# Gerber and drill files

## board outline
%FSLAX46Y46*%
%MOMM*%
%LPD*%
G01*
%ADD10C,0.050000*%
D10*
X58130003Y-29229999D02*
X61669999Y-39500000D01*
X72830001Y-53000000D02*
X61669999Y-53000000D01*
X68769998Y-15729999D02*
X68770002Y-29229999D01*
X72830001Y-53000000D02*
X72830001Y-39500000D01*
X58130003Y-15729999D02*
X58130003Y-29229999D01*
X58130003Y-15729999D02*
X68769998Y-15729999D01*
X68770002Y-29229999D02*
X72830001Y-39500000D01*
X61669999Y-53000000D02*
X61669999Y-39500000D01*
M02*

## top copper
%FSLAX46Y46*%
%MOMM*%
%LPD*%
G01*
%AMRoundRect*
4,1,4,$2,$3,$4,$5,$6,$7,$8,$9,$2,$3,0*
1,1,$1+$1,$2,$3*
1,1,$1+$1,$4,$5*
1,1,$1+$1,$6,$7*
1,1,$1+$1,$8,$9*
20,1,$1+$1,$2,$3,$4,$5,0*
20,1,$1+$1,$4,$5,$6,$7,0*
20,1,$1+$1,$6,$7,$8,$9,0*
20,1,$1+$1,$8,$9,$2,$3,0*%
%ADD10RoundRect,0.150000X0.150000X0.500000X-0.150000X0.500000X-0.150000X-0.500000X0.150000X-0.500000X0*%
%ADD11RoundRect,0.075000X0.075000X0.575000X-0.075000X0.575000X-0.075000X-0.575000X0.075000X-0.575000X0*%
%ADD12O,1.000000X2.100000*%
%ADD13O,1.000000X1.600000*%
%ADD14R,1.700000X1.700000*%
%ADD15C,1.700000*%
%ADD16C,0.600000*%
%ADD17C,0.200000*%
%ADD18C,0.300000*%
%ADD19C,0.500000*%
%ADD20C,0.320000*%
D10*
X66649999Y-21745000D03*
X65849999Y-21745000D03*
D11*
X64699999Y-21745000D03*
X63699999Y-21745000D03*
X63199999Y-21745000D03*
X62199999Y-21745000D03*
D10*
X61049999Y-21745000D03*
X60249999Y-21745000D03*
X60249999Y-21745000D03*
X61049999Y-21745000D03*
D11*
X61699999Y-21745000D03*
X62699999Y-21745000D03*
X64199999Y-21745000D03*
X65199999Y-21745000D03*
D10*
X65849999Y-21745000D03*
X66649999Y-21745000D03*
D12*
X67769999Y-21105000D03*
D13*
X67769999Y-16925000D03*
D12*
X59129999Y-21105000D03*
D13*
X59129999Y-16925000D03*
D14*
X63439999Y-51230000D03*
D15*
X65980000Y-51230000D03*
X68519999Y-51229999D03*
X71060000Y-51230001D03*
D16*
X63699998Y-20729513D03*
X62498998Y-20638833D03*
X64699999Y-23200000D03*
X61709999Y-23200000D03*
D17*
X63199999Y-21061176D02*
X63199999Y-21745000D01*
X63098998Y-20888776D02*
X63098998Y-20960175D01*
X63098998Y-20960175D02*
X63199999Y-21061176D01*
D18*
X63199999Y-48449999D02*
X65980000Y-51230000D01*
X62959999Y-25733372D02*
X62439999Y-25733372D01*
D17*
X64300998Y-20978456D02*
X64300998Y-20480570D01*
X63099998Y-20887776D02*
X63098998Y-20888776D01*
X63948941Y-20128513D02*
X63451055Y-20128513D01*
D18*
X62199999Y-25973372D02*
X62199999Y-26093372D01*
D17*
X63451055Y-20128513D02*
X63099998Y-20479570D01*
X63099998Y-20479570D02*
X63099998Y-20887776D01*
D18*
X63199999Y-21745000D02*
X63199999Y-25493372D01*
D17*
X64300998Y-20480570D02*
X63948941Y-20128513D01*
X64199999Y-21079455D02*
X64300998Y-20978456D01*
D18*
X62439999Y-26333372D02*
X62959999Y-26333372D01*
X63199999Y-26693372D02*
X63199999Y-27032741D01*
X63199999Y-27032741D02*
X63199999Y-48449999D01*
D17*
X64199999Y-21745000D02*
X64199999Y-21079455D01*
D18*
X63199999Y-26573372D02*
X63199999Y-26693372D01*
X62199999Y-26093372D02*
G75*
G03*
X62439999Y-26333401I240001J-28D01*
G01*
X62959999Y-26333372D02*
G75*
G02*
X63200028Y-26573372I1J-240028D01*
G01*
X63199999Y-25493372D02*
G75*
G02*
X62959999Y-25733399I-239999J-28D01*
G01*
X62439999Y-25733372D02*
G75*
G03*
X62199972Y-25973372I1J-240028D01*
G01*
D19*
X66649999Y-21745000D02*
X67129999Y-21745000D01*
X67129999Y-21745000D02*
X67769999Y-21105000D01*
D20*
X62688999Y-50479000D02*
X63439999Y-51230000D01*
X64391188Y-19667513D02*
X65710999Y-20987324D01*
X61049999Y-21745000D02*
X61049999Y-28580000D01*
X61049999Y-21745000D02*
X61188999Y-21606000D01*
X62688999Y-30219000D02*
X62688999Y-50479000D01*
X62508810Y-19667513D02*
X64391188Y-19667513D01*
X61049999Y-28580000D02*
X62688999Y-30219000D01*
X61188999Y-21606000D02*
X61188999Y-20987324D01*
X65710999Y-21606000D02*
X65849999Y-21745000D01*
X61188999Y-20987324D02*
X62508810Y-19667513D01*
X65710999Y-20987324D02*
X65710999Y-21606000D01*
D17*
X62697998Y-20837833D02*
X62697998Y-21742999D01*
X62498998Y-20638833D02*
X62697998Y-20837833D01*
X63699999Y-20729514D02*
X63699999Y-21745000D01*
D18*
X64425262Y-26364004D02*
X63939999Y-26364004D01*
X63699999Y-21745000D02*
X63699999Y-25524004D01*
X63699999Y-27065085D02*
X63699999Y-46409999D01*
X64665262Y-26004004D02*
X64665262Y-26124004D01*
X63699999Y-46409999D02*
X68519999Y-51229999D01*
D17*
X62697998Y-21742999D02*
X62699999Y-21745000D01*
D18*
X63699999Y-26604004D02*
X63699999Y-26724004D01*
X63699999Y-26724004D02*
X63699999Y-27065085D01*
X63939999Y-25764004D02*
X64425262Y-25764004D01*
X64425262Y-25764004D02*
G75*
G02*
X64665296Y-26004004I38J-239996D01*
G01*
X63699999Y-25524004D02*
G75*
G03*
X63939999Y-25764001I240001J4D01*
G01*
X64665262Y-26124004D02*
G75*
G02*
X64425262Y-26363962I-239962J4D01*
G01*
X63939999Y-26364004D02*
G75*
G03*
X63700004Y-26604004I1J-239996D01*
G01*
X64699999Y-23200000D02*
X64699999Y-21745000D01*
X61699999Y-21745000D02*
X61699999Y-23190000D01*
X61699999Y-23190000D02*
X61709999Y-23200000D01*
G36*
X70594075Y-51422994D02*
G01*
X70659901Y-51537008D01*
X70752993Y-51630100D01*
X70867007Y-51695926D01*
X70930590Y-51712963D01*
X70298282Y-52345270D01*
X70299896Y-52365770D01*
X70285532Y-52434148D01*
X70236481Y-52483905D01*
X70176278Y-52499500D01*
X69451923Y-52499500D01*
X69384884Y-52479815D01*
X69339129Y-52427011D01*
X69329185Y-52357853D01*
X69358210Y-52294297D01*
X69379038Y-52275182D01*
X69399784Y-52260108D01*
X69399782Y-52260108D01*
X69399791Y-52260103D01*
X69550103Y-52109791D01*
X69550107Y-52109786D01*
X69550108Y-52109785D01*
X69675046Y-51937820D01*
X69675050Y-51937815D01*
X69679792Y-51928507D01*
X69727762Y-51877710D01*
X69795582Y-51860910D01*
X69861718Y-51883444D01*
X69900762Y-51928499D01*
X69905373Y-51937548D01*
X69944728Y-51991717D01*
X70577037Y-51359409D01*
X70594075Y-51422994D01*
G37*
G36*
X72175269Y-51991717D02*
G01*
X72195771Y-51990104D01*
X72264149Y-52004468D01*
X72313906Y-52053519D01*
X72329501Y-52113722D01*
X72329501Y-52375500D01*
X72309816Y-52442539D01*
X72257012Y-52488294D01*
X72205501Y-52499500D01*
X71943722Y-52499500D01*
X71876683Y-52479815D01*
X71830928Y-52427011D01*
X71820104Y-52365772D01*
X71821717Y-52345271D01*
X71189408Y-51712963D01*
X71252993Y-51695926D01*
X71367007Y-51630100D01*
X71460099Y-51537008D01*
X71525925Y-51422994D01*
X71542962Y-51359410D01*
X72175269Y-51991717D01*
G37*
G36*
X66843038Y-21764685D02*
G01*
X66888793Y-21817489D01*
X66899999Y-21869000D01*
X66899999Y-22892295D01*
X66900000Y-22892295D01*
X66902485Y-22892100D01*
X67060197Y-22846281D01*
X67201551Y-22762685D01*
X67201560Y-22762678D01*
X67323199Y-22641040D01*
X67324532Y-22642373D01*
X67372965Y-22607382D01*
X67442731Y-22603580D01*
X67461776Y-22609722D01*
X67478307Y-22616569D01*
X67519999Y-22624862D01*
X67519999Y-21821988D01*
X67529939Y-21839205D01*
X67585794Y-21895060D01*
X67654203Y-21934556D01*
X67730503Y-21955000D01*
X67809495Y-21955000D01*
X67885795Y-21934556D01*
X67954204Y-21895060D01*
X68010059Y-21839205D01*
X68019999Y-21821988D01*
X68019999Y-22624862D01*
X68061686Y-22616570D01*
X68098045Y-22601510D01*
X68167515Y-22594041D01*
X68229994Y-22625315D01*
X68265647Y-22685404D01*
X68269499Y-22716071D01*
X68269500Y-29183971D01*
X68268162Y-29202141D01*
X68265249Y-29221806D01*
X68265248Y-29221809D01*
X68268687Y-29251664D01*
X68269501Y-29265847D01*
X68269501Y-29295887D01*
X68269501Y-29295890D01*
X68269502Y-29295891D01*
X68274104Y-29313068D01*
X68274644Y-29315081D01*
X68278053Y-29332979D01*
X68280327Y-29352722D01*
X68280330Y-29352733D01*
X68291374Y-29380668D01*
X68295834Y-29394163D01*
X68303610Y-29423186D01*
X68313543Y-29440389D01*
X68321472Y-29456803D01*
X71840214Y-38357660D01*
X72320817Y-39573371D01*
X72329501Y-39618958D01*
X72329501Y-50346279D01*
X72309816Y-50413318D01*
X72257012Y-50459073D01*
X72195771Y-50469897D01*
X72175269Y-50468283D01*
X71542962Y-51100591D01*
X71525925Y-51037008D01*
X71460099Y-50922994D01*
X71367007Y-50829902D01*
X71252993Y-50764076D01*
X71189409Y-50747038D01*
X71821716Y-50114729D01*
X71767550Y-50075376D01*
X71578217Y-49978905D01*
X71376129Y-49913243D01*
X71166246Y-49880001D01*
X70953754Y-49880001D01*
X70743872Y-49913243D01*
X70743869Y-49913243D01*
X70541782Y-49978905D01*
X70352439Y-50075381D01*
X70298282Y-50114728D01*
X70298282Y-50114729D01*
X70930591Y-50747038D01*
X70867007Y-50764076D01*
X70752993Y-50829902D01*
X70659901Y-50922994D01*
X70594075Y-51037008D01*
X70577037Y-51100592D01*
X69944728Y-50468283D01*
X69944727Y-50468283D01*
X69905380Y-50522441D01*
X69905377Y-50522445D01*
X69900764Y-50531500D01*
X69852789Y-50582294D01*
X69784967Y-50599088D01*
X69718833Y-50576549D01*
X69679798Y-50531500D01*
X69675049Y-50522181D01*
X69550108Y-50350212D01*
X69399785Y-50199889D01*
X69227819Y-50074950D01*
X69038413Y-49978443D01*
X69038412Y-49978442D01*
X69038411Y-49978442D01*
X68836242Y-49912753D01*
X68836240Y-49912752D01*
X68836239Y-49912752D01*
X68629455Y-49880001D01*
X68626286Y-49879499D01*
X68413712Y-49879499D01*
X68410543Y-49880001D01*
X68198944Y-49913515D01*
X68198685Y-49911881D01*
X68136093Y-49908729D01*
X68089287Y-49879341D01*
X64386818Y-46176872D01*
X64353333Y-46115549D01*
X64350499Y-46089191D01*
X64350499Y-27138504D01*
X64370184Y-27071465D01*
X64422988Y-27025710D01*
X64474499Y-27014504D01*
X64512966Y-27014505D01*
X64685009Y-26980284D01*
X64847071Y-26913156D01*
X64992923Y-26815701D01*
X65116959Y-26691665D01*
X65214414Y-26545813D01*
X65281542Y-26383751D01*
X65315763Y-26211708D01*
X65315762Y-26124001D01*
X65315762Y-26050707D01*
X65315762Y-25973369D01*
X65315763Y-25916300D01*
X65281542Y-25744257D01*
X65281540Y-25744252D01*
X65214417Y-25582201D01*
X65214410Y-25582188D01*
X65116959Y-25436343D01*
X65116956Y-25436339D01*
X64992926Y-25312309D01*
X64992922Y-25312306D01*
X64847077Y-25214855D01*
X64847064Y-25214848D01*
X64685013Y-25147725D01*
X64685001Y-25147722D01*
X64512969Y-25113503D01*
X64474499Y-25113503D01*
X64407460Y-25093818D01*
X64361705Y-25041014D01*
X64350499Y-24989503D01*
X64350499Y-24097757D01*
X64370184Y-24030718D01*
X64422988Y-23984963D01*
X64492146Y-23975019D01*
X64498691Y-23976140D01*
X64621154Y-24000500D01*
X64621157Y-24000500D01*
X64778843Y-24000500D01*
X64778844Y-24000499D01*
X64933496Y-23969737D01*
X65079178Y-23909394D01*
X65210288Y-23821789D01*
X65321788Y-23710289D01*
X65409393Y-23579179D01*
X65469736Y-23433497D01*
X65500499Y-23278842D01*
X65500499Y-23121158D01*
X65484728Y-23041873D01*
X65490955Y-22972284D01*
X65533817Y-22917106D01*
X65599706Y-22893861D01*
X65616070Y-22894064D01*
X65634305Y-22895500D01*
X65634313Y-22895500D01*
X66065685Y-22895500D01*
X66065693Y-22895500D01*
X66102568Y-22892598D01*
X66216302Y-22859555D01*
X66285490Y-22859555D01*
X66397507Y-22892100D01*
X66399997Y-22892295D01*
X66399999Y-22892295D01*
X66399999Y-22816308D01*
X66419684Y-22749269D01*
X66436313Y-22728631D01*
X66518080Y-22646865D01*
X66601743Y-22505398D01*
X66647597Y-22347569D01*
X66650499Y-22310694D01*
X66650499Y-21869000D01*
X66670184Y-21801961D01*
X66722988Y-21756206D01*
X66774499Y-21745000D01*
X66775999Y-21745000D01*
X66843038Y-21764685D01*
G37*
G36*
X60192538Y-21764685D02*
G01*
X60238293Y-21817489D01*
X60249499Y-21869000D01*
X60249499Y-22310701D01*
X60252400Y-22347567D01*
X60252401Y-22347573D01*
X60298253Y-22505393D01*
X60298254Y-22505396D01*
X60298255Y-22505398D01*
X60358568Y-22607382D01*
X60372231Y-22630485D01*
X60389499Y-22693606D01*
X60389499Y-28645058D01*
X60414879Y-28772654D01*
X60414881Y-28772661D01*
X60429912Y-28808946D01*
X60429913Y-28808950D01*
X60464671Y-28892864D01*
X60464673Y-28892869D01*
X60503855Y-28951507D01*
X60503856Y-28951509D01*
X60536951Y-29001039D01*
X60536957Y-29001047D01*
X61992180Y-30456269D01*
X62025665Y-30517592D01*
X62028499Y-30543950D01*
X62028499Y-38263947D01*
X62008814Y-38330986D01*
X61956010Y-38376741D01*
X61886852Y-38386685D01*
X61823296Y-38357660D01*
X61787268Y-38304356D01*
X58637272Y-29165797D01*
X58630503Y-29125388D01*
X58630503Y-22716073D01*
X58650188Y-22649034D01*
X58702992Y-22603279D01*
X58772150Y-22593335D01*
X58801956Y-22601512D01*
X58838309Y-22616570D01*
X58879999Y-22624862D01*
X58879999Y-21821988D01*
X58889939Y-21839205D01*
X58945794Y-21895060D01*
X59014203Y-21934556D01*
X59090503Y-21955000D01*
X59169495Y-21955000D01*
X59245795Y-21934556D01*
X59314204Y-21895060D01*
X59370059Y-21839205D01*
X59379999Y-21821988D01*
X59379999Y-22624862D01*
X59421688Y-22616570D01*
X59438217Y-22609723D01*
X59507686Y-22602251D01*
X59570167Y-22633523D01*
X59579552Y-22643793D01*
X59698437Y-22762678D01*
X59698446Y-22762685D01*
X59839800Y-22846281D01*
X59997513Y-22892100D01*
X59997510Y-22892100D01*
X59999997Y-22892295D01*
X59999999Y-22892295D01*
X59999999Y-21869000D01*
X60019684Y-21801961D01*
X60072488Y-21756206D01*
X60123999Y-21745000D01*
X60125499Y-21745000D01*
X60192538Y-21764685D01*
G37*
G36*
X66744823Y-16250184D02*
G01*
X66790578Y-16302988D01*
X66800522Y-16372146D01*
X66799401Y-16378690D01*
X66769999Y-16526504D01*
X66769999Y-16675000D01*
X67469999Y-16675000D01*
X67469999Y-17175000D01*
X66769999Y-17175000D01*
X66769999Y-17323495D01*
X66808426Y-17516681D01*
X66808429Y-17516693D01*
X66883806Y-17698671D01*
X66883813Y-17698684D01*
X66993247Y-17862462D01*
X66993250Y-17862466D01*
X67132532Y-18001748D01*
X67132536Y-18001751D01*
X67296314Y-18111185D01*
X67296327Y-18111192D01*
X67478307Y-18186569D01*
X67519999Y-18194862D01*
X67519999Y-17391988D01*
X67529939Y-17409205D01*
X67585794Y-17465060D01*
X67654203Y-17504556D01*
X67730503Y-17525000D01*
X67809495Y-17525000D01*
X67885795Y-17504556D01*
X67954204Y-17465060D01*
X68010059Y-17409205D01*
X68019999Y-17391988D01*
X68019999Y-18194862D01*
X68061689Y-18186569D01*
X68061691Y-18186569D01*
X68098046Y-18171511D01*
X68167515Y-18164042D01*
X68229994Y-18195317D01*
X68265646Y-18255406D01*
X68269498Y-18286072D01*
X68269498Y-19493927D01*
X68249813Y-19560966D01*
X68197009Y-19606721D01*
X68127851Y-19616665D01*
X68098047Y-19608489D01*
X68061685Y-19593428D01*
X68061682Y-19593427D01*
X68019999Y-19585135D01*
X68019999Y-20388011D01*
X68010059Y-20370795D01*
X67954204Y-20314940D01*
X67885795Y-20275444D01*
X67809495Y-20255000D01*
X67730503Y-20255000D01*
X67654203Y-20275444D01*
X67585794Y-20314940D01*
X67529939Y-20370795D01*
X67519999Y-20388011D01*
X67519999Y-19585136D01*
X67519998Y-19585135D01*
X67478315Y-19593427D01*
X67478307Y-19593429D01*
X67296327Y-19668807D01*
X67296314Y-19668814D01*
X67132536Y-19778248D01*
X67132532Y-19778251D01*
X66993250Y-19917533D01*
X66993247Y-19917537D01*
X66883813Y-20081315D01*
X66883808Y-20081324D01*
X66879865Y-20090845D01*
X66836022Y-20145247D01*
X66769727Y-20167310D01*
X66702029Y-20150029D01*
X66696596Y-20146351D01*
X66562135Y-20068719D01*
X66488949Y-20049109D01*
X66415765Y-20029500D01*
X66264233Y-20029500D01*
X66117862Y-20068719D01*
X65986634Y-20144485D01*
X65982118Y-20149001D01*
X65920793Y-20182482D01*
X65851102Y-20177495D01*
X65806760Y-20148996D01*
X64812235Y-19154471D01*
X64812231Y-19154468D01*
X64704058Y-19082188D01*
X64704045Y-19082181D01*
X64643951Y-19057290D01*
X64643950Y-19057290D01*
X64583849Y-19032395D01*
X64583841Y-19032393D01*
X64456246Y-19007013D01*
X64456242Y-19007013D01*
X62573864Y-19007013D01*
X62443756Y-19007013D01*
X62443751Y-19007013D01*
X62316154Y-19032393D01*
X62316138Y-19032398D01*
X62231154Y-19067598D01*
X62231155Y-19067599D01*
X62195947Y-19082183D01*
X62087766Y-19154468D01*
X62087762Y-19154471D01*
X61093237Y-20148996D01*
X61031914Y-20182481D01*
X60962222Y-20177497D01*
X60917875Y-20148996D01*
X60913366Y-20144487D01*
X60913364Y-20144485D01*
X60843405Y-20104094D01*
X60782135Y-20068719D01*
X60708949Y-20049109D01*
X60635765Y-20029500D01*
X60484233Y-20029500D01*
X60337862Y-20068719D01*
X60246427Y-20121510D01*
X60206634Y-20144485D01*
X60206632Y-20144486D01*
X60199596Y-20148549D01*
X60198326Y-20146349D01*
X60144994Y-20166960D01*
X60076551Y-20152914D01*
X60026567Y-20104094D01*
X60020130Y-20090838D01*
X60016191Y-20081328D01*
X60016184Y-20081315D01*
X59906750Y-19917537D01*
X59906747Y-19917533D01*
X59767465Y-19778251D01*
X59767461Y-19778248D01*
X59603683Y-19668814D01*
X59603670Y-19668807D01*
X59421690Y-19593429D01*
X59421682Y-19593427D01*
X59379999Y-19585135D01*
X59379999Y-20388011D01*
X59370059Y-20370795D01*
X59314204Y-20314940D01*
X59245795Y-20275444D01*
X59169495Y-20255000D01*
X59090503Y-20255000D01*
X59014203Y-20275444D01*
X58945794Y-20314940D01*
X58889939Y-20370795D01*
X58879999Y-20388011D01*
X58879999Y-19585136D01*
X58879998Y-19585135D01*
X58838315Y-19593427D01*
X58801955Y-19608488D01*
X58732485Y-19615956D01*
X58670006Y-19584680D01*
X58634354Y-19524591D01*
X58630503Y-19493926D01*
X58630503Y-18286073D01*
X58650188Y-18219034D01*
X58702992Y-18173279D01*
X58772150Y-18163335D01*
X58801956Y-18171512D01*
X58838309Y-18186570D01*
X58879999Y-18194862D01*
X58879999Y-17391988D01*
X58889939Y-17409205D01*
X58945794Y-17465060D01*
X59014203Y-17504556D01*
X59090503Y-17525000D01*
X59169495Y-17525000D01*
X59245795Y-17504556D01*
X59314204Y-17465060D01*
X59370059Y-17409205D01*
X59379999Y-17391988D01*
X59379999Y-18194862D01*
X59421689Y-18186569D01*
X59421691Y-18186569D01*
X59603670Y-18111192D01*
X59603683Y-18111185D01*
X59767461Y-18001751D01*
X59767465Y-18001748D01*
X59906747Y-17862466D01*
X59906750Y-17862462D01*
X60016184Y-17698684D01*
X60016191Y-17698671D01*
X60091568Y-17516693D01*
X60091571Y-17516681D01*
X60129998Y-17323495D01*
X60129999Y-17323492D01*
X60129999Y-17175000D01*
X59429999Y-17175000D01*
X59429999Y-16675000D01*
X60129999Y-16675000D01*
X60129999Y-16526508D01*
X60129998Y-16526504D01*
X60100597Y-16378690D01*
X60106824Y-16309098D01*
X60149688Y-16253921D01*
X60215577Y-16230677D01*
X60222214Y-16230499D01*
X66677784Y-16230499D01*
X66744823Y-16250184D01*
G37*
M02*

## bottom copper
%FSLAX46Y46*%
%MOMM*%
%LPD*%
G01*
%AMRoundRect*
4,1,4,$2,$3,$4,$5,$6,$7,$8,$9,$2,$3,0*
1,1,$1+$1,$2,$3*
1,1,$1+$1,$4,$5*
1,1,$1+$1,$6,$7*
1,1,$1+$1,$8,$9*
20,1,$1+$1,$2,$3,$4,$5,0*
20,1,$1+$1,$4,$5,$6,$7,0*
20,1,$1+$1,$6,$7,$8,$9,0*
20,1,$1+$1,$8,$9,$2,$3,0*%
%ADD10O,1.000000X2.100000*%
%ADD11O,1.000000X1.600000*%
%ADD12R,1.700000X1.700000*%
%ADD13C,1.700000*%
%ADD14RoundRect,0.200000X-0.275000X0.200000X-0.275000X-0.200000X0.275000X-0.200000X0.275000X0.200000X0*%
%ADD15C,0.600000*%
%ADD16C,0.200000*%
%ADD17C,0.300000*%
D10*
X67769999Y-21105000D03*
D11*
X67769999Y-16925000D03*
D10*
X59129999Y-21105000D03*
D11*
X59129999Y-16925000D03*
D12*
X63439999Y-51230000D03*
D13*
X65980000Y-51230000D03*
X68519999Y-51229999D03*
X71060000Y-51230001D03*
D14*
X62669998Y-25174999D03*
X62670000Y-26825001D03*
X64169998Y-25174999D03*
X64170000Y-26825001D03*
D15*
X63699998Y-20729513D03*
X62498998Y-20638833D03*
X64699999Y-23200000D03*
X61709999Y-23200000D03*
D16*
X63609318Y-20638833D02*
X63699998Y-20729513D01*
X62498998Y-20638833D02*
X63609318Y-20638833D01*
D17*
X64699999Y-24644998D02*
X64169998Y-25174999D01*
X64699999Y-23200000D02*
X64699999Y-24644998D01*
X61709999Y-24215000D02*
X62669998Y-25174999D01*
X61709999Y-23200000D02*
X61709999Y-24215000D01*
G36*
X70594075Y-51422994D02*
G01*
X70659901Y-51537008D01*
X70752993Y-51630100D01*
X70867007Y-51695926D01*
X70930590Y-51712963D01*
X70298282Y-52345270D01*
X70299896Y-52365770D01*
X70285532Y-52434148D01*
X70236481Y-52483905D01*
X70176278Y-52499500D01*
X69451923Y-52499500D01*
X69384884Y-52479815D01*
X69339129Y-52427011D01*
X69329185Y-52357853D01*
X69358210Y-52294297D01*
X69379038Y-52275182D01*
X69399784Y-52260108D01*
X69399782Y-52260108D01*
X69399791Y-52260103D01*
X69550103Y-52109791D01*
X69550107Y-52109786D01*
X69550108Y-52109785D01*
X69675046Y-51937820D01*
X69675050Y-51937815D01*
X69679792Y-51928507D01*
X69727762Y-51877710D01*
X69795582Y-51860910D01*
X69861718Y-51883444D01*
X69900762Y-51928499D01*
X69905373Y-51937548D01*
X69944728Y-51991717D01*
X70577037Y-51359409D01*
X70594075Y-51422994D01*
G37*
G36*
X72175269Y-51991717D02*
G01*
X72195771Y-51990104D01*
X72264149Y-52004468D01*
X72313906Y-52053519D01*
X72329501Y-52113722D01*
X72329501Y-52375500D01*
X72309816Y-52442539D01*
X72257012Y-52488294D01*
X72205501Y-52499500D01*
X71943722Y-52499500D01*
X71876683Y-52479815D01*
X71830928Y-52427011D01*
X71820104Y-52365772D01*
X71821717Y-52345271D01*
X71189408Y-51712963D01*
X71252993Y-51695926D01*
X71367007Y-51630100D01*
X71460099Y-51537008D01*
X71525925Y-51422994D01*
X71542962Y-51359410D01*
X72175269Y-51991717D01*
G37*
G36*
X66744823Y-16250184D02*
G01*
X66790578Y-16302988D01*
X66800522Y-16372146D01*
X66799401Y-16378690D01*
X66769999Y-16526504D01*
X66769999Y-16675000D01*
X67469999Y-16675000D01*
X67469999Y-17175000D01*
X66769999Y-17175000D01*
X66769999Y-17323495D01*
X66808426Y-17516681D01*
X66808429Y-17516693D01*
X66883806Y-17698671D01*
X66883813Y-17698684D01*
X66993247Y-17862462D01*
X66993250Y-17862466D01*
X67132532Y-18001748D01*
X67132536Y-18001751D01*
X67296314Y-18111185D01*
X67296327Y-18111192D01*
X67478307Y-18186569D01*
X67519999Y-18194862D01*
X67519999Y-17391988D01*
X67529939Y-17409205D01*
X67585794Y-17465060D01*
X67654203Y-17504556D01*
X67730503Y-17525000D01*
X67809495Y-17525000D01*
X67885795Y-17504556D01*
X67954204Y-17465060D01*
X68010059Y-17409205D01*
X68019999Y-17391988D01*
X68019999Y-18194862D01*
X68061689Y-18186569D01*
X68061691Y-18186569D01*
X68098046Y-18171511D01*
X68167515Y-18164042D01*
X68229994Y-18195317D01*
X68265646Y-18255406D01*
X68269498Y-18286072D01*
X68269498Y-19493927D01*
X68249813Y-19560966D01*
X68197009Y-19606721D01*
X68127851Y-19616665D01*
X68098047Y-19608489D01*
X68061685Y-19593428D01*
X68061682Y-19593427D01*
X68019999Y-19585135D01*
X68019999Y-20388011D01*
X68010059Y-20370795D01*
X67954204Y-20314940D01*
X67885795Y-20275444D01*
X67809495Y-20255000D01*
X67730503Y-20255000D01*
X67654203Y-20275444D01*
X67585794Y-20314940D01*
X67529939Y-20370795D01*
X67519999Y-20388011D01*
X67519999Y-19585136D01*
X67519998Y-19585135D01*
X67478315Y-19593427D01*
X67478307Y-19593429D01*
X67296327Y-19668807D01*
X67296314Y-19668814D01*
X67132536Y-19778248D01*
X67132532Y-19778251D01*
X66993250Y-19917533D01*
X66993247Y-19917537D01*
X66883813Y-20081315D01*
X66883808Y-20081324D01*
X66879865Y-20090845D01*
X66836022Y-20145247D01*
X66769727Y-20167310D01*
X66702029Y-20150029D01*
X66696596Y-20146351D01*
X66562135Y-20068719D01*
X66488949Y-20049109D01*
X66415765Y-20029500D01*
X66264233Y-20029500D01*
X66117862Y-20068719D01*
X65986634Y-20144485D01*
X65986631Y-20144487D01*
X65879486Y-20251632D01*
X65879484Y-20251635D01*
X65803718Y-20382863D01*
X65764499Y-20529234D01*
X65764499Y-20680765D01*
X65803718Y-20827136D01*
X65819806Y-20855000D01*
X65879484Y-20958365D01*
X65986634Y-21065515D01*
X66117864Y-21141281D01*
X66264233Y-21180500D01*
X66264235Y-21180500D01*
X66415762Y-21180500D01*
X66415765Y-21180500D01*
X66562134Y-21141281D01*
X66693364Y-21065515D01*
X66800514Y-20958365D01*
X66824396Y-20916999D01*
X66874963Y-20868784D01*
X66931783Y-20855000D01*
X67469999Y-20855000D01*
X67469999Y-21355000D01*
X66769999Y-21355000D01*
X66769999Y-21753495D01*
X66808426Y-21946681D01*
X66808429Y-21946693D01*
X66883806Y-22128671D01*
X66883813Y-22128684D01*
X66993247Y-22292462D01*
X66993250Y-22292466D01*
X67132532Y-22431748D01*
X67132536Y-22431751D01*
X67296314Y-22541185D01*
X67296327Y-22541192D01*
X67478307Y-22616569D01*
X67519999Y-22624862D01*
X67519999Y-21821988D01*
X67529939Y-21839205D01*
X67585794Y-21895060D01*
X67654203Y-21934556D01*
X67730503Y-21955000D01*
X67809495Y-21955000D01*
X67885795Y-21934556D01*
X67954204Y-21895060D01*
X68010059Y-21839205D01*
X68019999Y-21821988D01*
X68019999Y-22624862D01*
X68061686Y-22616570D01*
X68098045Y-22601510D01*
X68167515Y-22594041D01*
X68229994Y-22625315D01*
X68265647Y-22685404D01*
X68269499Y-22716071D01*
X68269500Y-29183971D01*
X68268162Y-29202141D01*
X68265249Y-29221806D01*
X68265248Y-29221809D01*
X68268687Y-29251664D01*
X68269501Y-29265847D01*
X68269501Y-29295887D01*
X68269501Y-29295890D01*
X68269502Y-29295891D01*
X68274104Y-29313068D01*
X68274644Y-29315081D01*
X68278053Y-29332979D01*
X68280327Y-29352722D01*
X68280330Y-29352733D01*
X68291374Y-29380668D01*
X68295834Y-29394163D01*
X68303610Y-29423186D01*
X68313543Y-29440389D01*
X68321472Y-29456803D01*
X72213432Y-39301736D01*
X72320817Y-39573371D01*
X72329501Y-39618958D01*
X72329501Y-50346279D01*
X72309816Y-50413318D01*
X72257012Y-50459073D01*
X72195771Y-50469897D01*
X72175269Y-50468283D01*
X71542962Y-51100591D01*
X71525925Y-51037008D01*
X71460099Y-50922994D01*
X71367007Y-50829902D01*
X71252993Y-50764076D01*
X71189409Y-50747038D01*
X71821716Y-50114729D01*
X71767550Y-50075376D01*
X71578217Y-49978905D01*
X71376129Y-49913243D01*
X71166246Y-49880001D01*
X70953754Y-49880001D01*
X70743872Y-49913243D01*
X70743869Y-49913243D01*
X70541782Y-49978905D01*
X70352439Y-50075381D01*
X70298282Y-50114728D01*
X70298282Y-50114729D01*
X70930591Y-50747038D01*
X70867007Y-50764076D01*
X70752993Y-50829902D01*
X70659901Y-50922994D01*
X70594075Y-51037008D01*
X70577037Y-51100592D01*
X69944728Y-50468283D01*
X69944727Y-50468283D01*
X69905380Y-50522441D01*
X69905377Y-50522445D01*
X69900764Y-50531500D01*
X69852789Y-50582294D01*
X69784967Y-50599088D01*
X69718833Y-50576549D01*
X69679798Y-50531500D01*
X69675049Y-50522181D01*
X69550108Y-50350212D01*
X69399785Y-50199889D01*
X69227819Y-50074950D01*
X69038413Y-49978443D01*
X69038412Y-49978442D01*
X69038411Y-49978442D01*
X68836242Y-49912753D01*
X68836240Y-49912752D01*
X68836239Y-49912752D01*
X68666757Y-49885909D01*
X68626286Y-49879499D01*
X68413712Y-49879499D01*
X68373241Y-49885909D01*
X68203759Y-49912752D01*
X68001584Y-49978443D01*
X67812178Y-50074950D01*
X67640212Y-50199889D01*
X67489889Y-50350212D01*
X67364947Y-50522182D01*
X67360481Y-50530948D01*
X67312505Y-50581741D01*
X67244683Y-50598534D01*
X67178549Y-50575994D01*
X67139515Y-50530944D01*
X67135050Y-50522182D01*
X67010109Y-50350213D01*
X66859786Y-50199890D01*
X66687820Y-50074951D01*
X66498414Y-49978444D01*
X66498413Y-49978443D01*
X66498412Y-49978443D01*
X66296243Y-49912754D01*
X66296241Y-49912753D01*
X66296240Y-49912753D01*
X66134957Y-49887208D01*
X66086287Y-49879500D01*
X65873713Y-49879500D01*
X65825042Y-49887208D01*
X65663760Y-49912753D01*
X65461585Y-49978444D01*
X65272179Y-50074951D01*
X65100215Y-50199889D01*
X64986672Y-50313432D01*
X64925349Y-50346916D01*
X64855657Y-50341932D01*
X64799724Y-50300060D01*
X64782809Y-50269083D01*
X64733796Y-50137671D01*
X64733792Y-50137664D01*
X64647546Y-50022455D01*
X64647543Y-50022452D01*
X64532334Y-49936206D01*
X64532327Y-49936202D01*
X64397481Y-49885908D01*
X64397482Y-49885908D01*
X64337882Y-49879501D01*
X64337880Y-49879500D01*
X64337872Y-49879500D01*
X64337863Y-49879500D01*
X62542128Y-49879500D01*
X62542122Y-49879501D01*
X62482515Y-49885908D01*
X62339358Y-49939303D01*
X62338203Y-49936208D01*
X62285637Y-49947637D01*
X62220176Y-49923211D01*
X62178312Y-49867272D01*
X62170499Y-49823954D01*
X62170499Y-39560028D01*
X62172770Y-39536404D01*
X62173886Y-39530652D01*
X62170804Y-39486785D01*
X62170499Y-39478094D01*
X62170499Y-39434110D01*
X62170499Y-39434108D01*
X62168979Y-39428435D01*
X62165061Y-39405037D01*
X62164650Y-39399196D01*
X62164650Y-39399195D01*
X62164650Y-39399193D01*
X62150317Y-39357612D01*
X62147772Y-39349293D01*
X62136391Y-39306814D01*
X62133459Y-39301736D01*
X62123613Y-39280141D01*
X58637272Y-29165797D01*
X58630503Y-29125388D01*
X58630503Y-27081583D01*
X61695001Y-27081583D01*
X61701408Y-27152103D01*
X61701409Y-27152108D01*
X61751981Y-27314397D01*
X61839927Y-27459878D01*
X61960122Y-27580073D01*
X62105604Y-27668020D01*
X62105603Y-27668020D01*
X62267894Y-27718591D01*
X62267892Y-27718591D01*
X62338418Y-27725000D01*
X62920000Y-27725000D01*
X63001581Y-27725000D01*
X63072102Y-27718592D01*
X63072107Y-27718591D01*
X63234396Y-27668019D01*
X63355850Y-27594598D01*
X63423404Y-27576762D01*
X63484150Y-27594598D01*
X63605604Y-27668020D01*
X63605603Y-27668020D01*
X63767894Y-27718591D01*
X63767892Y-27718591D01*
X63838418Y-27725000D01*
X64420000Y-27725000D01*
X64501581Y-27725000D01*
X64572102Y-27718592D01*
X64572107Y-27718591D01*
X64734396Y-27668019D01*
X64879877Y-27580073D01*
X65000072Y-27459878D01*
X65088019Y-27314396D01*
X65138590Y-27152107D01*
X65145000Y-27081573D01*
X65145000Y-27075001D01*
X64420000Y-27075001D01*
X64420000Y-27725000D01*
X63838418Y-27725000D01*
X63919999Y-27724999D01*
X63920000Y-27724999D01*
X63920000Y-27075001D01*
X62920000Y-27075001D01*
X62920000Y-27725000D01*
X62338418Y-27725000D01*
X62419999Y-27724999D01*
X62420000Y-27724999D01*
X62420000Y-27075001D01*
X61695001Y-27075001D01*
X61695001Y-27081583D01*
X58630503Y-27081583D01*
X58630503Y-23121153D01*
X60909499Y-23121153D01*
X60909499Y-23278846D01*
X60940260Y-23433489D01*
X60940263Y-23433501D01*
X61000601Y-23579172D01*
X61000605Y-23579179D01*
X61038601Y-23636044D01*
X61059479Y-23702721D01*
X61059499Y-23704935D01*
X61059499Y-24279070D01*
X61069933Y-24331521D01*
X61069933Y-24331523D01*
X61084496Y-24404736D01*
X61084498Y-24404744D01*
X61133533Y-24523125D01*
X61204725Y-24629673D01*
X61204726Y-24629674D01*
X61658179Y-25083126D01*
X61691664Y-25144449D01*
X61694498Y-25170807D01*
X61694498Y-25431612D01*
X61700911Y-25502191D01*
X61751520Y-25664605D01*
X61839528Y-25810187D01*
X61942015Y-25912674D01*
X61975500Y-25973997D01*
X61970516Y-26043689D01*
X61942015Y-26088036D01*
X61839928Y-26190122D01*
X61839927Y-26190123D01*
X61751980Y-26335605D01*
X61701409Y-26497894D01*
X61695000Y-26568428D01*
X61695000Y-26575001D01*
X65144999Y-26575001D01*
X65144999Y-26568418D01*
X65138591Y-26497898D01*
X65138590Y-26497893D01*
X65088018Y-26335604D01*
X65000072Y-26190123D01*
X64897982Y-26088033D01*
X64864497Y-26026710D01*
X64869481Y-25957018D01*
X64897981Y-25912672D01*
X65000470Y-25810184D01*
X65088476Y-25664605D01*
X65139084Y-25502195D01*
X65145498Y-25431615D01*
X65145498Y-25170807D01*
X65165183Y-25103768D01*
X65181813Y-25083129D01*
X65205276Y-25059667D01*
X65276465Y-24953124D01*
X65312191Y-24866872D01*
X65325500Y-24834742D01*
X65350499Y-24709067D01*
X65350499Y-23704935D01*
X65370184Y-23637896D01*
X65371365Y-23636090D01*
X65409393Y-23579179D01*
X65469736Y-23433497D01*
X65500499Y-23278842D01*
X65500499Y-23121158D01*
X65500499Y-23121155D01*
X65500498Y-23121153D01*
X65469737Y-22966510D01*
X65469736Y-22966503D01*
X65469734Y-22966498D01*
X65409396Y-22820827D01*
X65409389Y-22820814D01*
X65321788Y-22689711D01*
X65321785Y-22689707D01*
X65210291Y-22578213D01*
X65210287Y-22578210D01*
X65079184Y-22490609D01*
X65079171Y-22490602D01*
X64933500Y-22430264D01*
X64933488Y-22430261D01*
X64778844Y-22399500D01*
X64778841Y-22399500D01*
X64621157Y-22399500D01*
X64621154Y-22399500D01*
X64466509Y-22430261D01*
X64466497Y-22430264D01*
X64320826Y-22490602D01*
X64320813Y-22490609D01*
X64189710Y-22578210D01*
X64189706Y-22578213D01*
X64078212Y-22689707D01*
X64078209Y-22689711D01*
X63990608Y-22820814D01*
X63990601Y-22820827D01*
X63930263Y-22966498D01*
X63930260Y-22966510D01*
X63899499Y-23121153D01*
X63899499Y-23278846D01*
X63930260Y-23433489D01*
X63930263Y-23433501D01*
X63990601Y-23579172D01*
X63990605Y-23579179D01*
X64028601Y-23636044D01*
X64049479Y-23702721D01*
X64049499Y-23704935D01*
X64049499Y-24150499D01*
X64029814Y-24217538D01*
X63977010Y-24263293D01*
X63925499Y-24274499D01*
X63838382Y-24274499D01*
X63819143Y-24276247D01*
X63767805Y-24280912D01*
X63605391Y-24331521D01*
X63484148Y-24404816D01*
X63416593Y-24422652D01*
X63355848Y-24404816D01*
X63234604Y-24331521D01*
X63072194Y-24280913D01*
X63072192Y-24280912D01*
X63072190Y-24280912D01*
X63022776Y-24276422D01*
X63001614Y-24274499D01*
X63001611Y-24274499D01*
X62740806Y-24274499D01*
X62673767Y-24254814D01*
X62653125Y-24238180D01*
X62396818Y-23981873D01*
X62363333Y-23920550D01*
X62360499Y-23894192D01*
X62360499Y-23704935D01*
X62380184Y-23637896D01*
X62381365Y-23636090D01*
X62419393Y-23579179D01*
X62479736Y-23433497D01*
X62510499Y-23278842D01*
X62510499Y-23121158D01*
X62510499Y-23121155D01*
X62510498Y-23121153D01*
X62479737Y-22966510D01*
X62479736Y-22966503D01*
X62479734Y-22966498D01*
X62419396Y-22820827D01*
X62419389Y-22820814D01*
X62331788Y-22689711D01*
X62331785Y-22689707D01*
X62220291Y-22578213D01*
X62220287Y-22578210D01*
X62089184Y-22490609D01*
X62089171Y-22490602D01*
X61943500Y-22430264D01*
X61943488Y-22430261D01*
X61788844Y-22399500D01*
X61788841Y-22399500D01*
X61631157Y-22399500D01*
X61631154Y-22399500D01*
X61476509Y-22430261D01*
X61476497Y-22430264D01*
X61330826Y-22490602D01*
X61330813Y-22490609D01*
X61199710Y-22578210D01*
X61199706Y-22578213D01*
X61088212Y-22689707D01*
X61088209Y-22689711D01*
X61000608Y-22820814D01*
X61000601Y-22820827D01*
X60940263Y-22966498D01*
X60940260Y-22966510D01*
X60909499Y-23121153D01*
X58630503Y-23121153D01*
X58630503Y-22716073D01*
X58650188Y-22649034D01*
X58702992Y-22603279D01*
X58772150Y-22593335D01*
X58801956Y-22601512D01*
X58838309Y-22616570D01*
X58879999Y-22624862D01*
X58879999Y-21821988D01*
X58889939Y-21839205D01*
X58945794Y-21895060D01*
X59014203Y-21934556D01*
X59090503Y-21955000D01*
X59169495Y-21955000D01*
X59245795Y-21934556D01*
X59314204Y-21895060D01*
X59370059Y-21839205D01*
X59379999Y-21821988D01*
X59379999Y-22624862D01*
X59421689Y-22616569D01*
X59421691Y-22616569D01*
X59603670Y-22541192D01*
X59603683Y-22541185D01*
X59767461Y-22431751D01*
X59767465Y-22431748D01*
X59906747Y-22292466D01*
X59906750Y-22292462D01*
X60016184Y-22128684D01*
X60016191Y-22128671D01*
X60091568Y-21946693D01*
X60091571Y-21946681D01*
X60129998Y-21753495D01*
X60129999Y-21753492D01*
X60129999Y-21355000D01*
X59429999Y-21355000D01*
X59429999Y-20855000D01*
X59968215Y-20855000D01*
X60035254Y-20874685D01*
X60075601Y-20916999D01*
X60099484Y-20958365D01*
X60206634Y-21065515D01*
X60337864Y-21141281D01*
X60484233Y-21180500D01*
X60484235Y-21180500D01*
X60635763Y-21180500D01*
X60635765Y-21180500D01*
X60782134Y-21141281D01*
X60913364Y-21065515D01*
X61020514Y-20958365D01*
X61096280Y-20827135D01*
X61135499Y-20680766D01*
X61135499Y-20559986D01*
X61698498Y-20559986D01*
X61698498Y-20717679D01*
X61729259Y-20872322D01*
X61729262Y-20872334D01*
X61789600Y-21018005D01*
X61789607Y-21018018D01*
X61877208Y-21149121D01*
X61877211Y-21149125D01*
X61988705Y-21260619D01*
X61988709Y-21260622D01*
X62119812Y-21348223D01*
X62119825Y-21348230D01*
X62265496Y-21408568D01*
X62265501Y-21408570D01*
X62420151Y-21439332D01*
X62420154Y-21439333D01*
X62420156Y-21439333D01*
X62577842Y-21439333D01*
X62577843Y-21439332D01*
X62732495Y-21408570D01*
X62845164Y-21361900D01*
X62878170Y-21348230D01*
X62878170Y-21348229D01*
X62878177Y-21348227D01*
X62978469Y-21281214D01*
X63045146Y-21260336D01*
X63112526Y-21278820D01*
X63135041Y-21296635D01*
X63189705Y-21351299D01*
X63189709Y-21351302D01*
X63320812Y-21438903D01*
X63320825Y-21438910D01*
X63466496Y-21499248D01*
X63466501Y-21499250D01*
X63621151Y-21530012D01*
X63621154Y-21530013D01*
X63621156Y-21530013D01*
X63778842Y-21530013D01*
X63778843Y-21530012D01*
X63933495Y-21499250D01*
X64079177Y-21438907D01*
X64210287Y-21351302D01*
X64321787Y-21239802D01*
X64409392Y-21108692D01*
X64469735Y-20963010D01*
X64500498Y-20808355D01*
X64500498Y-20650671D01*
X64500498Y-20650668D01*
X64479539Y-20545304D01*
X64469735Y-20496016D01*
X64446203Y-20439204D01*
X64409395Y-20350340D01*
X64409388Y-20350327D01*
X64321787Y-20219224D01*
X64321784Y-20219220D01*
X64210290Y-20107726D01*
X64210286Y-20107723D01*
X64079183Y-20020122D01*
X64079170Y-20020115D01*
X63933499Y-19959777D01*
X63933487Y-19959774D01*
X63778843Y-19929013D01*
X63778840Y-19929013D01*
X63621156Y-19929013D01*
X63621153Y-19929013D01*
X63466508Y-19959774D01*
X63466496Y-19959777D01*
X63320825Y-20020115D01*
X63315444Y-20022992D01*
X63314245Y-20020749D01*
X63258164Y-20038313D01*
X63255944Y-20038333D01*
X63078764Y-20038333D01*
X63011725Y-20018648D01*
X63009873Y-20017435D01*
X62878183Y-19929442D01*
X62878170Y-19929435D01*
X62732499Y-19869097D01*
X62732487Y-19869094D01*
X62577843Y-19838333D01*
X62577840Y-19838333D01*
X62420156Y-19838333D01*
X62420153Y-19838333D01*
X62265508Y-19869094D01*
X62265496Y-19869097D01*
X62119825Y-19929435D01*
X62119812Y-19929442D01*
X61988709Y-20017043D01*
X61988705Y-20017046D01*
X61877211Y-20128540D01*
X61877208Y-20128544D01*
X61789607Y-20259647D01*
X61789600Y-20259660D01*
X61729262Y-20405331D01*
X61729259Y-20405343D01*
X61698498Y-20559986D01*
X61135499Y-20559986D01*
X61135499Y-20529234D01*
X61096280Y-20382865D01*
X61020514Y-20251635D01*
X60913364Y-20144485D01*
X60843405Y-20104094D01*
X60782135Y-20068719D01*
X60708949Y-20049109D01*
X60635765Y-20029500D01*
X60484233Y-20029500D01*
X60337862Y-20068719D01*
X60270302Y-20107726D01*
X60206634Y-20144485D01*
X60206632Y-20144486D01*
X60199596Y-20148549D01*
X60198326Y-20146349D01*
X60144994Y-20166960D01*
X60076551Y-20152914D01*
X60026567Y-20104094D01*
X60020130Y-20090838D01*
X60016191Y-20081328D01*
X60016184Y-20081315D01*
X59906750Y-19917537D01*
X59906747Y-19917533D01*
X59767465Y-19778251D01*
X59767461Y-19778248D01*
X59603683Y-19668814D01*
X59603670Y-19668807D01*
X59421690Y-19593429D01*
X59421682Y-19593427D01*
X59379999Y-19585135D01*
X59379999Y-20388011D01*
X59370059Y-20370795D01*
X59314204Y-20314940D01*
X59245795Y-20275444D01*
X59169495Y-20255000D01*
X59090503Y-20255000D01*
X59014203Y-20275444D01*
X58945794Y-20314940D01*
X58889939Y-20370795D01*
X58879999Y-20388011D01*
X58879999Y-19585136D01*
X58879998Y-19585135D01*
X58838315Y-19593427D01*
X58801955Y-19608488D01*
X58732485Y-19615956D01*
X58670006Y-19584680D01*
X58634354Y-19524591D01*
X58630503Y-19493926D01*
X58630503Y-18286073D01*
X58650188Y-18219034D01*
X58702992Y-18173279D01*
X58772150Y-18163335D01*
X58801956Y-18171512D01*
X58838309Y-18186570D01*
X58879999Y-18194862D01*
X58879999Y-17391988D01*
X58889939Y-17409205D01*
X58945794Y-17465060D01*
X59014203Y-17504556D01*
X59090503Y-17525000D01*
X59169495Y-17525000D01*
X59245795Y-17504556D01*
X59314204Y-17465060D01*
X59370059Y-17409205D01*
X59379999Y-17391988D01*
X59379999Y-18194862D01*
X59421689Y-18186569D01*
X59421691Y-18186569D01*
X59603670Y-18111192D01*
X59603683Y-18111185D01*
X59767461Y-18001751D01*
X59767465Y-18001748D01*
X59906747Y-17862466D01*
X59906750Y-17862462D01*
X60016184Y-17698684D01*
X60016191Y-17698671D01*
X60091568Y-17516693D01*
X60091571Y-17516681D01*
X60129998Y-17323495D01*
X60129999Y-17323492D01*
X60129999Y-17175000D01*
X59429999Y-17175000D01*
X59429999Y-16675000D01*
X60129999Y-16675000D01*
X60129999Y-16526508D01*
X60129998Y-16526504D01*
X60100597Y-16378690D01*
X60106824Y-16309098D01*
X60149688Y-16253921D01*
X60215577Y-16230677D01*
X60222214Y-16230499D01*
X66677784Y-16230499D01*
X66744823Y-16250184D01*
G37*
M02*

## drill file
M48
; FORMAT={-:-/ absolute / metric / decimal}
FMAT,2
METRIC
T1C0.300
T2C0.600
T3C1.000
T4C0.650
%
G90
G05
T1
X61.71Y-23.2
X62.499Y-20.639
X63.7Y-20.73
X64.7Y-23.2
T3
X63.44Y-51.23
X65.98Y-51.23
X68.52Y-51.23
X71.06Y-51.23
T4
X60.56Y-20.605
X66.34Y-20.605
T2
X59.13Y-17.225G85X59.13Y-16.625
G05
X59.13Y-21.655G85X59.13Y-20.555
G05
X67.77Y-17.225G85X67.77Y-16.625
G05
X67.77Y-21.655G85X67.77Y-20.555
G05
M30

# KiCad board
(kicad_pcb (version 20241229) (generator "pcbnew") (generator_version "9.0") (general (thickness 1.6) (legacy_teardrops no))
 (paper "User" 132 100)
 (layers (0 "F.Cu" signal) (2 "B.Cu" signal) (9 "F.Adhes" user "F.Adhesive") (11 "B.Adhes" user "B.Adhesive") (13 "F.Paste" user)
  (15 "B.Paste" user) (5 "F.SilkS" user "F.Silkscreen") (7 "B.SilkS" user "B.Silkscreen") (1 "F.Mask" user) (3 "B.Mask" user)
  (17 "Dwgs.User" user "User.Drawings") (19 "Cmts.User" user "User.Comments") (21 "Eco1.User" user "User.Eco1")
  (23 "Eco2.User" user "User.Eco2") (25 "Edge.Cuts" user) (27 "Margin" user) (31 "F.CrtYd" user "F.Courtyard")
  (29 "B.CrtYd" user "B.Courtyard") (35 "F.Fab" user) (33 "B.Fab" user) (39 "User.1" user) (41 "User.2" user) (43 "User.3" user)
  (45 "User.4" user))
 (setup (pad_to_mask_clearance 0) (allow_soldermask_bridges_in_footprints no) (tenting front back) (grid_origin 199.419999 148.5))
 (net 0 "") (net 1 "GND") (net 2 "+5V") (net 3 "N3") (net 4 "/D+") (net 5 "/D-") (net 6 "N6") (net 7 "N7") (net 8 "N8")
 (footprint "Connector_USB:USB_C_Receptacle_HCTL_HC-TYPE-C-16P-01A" (layer "F.Cu") (at 63.449999 18 180)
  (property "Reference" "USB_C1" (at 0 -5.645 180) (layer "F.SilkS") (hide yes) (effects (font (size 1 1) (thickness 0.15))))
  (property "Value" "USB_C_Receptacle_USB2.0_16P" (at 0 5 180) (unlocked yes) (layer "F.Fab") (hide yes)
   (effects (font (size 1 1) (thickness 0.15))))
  (pad "" np_thru_hole circle (at -2.89 -2.605 180) (size 0.65 0.65) (drill 0.65) (layers "*.Mask"))
  (pad "" np_thru_hole circle (at 2.89 -2.605 180) (size 0.65 0.65) (drill 0.65) (layers "*.Mask"))
  (pad "A1" smd roundrect (at -3.2 -3.745 180) (size 0.6 1.3) (layers "F.Cu" "F.Mask" "F.Paste") (roundrect_rratio 0.25) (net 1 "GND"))
  (pad "A4" smd roundrect (at -2.4 -3.745 180) (size 0.6 1.3) (layers "F.Cu" "F.Mask" "F.Paste") (roundrect_rratio 0.25) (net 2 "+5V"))
  (pad "A5" smd roundrect (at -1.25 -3.745 180) (size 0.3 1.3) (layers "F.Cu" "F.Mask" "F.Paste") (roundrect_rratio 0.25) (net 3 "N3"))
  (pad "A6" smd roundrect (at -0.25 -3.745 180) (size 0.3 1.3) (layers "F.Cu" "F.Mask" "F.Paste") (roundrect_rratio 0.25) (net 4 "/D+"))
  (pad "A7" smd roundrect (at 0.25 -3.745 180) (size 0.3 1.3) (layers "F.Cu" "F.Mask" "F.Paste") (roundrect_rratio 0.25) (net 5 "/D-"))
  (pad "A8" smd roundrect (at 1.25 -3.745 180) (size 0.3 1.3) (layers "F.Cu" "F.Mask" "F.Paste") (roundrect_rratio 0.25) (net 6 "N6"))
  (pad "A9" smd roundrect (at 2.4 -3.745 180) (size 0.6 1.3) (layers "F.Cu" "F.Mask" "F.Paste") (roundrect_rratio 0.25) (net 2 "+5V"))
  (pad "A12" smd roundrect (at 3.2 -3.745 180) (size 0.6 1.3) (layers "F.Cu" "F.Mask" "F.Paste") (roundrect_rratio 0.25) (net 1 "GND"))
  (pad "B1" smd roundrect (at 3.2 -3.745 180) (size 0.6 1.3) (layers "F.Cu" "F.Mask" "F.Paste") (roundrect_rratio 0.25) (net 1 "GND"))
  (pad "B4" smd roundrect (at 2.4 -3.745 180) (size 0.6 1.3) (layers "F.Cu" "F.Mask" "F.Paste") (roundrect_rratio 0.25) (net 2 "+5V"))
  (pad "B5" smd roundrect (at 1.75 -3.745 180) (size 0.3 1.3) (layers "F.Cu" "F.Mask" "F.Paste") (roundrect_rratio 0.25) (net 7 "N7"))
  (pad "B6" smd roundrect (at 0.75 -3.745 180) (size 0.3 1.3) (layers "F.Cu" "F.Mask" "F.Paste") (roundrect_rratio 0.25) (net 4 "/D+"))
  (pad "B7" smd roundrect (at -0.75 -3.745 180) (size 0.3 1.3) (layers "F.Cu" "F.Mask" "F.Paste") (roundrect_rratio 0.25) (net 5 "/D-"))
  (pad "B8" smd roundrect (at -1.75 -3.745 180) (size 0.3 1.3) (layers "F.Cu" "F.Mask" "F.Paste") (roundrect_rratio 0.25) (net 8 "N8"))
  (pad "B9" smd roundrect (at -2.4 -3.745 180) (size 0.6 1.3) (layers "F.Cu" "F.Mask" "F.Paste") (roundrect_rratio 0.25) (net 2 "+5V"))
  (pad "B12" smd roundrect (at -3.2 -3.745 180) (size 0.6 1.3) (layers "F.Cu" "F.Mask" "F.Paste") (roundrect_rratio 0.25) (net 1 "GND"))
  (pad "S1" thru_hole oval (at -4.32 -3.105 180) (size 1 2.1) (drill oval 0.6 1.7) (layers "*.Cu" "*.Mask") (remove_unused_layers no)
   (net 1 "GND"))
  (pad "S1" thru_hole oval (at -4.32 1.075 180) (size 1 1.6) (drill oval 0.6 1.2) (layers "*.Cu" "*.Mask") (remove_unused_layers no)
   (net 1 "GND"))
  (pad "S1" thru_hole oval (at 4.32 -3.105 180) (size 1 2.1) (drill oval 0.6 1.7) (layers "*.Cu" "*.Mask") (remove_unused_layers no)
   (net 1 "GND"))
  (pad "S1" thru_hole oval (at 4.32 1.075 180) (size 1 1.6) (drill oval 0.6 1.2) (layers "*.Cu" "*.Mask") (remove_unused_layers no)
   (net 1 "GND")))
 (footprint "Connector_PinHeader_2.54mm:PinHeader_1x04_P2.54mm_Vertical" (layer "F.Cu") (at 63.439999 51.23 90)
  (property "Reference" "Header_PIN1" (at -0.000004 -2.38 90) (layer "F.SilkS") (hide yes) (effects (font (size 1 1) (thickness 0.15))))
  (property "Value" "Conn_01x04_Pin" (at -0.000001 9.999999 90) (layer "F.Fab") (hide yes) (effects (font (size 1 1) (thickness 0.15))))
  (pad "1" thru_hole rect (at 0 0 90) (size 1.7 1.7) (drill 1) (layers "*.Cu" "*.Mask") (remove_unused_layers no) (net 2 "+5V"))
  (pad "2" thru_hole circle (at 0 2.540001 90) (size 1.7 1.7) (drill 1) (layers "*.Cu" "*.Mask") (remove_unused_layers no) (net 5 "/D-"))
  (pad "3" thru_hole circle (at 0.000001 5.08 90) (size 1.7 1.7) (drill 1) (layers "*.Cu" "*.Mask") (remove_unused_layers no) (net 4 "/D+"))
  (pad "4" thru_hole circle (at -0.000001 7.620001 90) (size 1.7 1.7) (drill 1) (layers "*.Cu" "*.Mask") (remove_unused_layers no)
   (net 1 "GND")))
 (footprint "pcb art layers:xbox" (layer "F.Cu") (at 65.419999 34.5)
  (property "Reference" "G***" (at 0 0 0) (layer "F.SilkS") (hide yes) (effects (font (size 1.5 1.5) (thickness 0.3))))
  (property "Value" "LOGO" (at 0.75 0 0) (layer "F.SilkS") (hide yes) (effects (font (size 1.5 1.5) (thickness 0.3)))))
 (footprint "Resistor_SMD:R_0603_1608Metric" (layer "B.Cu") (at 62.669999 26 -90)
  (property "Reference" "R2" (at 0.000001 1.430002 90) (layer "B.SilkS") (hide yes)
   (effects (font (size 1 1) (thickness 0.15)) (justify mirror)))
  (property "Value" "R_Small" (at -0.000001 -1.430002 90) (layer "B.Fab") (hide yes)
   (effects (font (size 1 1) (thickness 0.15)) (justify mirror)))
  (pad "1" smd roundrect (at -0.825001 0.000001 270) (size 0.8 0.95) (layers "B.Cu" "B.Mask" "B.Paste") (roundrect_rratio 0.25) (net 7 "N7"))
  (pad "2" smd roundrect (at 0.825001 -0.000001 270) (size 0.8 0.95) (layers "B.Cu" "B.Mask" "B.Paste") (roundrect_rratio 0.25)
   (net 1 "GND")))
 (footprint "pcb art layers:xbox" (layer "B.Cu") (at 65.419999 34.5 180)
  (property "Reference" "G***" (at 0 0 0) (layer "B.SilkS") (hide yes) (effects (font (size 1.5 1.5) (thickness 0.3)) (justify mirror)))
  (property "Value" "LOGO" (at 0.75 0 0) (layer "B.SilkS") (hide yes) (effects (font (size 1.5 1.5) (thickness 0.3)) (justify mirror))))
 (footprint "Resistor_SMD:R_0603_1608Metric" (layer "B.Cu") (at 64.169999 26 -90)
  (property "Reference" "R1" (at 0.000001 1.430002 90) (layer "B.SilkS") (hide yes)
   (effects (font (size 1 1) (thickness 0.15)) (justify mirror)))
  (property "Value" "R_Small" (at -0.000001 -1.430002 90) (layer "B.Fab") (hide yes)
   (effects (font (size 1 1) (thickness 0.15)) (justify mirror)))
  (pad "1" smd roundrect (at -0.825001 0.000001 270) (size 0.8 0.95) (layers "B.Cu" "B.Mask" "B.Paste") (roundrect_rratio 0.25) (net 3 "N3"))
  (pad "2" smd roundrect (at 0.825001 -0.000001 270) (size 0.8 0.95) (layers "B.Cu" "B.Mask" "B.Paste") (roundrect_rratio 0.25)
   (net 1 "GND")))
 (gr_line (start 58.130003 29.229999) (end 61.669999 39.5) (stroke (width 0.05) (type default)) (layer "Edge.Cuts"))
 (gr_line (start 72.830001 53) (end 61.669999 53) (stroke (width 0.05) (type default)) (layer "Edge.Cuts"))
 (gr_line (start 68.769998 15.729999) (end 68.770002 29.229999) (stroke (width 0.05) (type default)) (layer "Edge.Cuts"))
 (gr_line (start 72.830001 53) (end 72.830001 39.5) (stroke (width 0.05) (type default)) (layer "Edge.Cuts"))
 (gr_line (start 58.130003 15.729999) (end 58.130003 29.229999) (stroke (width 0.05) (type default)) (layer "Edge.Cuts"))
 (gr_line (start 58.130003 15.729999) (end 68.769998 15.729999) (stroke (width 0.05) (type default)) (layer "Edge.Cuts"))
 (gr_line (start 68.770002 29.229999) (end 72.830001 39.5) (stroke (width 0.05) (type default)) (layer "Edge.Cuts"))
 (gr_line (start 61.669999 53) (end 61.669999 39.5) (stroke (width 0.05) (type default)) (layer "Edge.Cuts"))
 (segment (start 63.199999 21.061176) (end 63.199999 21.745) (width 0.2) (layer "F.Cu") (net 5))
 (segment (start 63.098998 20.888776) (end 63.098998 20.960175) (width 0.2) (layer "F.Cu") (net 5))
 (segment (start 63.098998 20.960175) (end 63.199999 21.061176) (width 0.2) (layer "F.Cu") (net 5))
 (segment (start 63.199999 48.449999) (end 65.98 51.23) (width 0.3) (layer "F.Cu") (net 5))
 (segment (start 62.959999 25.733372) (end 62.439999 25.733372) (width 0.3) (layer "F.Cu") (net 5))
 (segment (start 64.300998 20.978456) (end 64.300998 20.48057) (width 0.2) (layer "F.Cu") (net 5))
 (segment (start 63.099998 20.887776) (end 63.098998 20.888776) (width 0.2) (layer "F.Cu") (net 5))
 (segment (start 63.948941 20.128513) (end 63.451055 20.128513) (width 0.2) (layer "F.Cu") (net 5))
 (segment (start 62.199999 25.973372) (end 62.199999 26.093372) (width 0.3) (layer "F.Cu") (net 5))
 (segment (start 63.451055 20.128513) (end 63.099998 20.47957) (width 0.2) (layer "F.Cu") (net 5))
 (segment (start 63.099998 20.47957) (end 63.099998 20.887776) (width 0.2) (layer "F.Cu") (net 5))
 (segment (start 63.199999 21.745) (end 63.199999 25.493372) (width 0.3) (layer "F.Cu") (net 5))
 (segment (start 64.300998 20.48057) (end 63.948941 20.128513) (width 0.2) (layer "F.Cu") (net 5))
 (segment (start 64.199999 21.079455) (end 64.300998 20.978456) (width 0.2) (layer "F.Cu") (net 5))
 (segment (start 62.439999 26.333372) (end 62.959999 26.333372) (width 0.3) (layer "F.Cu") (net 5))
 (segment (start 63.199999 26.693372) (end 63.199999 27.032741) (width 0.3) (layer "F.Cu") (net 5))
 (segment (start 63.199999 27.032741) (end 63.199999 48.449999) (width 0.3) (layer "F.Cu") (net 5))
 (segment (start 64.199999 21.745) (end 64.199999 21.079455) (width 0.2) (layer "F.Cu") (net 5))
 (segment (start 63.199999 26.573372) (end 63.199999 26.693372) (width 0.3) (layer "F.Cu") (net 5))
 (arc (start 62.199999 26.093372) (mid 62.270293 26.263078) (end 62.439999 26.333372) (width 0.3) (layer "F.Cu") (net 5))
 (arc (start 62.959999 26.333372) (mid 63.129705 26.403666) (end 63.199999 26.573372) (width 0.3) (layer "F.Cu") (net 5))
 (arc (start 63.199999 25.493372) (mid 63.129705 25.663078) (end 62.959999 25.733372) (width 0.3) (layer "F.Cu") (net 5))
 (arc (start 62.439999 25.733372) (mid 62.270293 25.803666) (end 62.199999 25.973372) (width 0.3) (layer "F.Cu") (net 5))
 (segment (start 66.649999 21.745) (end 67.129999 21.745) (width 0.5) (layer "F.Cu") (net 1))
 (segment (start 67.129999 21.745) (end 67.769999 21.105) (width 0.5) (layer "F.Cu") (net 1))
 (segment (start 62.688999 50.479) (end 63.439999 51.23) (width 0.32) (layer "F.Cu") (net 2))
 (segment (start 64.391188 19.667513) (end 65.710999 20.987324) (width 0.32) (layer "F.Cu") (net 2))
 (segment (start 61.049999 21.745) (end 61.049999 28.58) (width 0.32) (layer "F.Cu") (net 2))
 (segment (start 61.049999 21.745) (end 61.188999 21.606) (width 0.32) (layer "F.Cu") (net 2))
 (segment (start 62.688999 30.219) (end 62.688999 50.479) (width 0.32) (layer "F.Cu") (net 2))
 (segment (start 62.50881 19.667513) (end 64.391188 19.667513) (width 0.32) (layer "F.Cu") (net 2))
 (segment (start 61.049999 28.58) (end 62.688999 30.219) (width 0.32) (layer "F.Cu") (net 2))
 (segment (start 61.188999 21.606) (end 61.188999 20.987324) (width 0.32) (layer "F.Cu") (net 2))
 (segment (start 65.710999 21.606) (end 65.849999 21.745) (width 0.32) (layer "F.Cu") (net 2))
 (segment (start 61.188999 20.987324) (end 62.50881 19.667513) (width 0.32) (layer "F.Cu") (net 2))
 (segment (start 65.710999 20.987324) (end 65.710999 21.606) (width 0.32) (layer "F.Cu") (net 2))
 (segment (start 62.697998 20.837833) (end 62.697998 21.742999) (width 0.2) (layer "F.Cu") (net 4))
 (segment (start 62.498998 20.638833) (end 62.697998 20.837833) (width 0.2) (layer "F.Cu") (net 4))
 (segment (start 63.699999 20.729514) (end 63.699999 21.745) (width 0.2) (layer "F.Cu") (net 4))
 (segment (start 64.425262 26.364004) (end 63.939999 26.364004) (width 0.3) (layer "F.Cu") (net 4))
 (segment (start 63.699999 21.745) (end 63.699999 25.524004) (width 0.3) (layer "F.Cu") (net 4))
 (segment (start 63.699999 27.065085) (end 63.699999 46.409999) (width 0.3) (layer "F.Cu") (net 4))
 (segment (start 64.665262 26.004004) (end 64.665262 26.124004) (width 0.3) (layer "F.Cu") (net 4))
 (segment (start 63.699999 46.409999) (end 68.519999 51.229999) (width 0.3) (layer "F.Cu") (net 4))
 (segment (start 62.697998 21.742999) (end 62.699999 21.745) (width 0.2) (layer "F.Cu") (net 4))
 (segment (start 63.699999 26.604004) (end 63.699999 26.724004) (width 0.3) (layer "F.Cu") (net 4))
 (segment (start 63.699999 26.724004) (end 63.699999 27.065085) (width 0.3) (layer "F.Cu") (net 4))
 (segment (start 63.939999 25.764004) (end 64.425262 25.764004) (width 0.3) (layer "F.Cu") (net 4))
 (via (at 63.699998 20.729513) (size 0.6) (drill 0.3) (layers "F.Cu" "B.Cu") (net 4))
 (via (at 62.498998 20.638833) (size 0.6) (drill 0.3) (layers "F.Cu" "B.Cu") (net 4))
 (arc (start 64.425262 25.764004) (mid 64.594968 25.834298) (end 64.665262 26.004004) (width 0.3) (layer "F.Cu") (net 4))
 (arc (start 63.699999 25.524004) (mid 63.770293 25.69371) (end 63.939999 25.764004) (width 0.3) (layer "F.Cu") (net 4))
 (arc (start 64.665262 26.124004) (mid 64.594968 26.29371) (end 64.425262 26.364004) (width 0.3) (layer "F.Cu") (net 4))
 (arc (start 63.939999 26.364004) (mid 63.770293 26.434298) (end 63.699999 26.604004) (width 0.3) (layer "F.Cu") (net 4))
 (segment (start 63.609318 20.638833) (end 63.699998 20.729513) (width 0.2) (layer "B.Cu") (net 4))
 (segment (start 62.498998 20.638833) (end 63.609318 20.638833) (width 0.2) (layer "B.Cu") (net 4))
 (segment (start 64.699999 23.2) (end 64.699999 21.745) (width 0.3) (layer "F.Cu") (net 3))
 (via (at 64.699999 23.2) (size 0.6) (drill 0.3) (layers "F.Cu" "B.Cu") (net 3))
 (segment (start 64.699999 24.644998) (end 64.169998 25.174999) (width 0.3) (layer "B.Cu") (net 3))
 (segment (start 64.699999 23.2) (end 64.699999 24.644998) (width 0.3) (layer "B.Cu") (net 3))
 (segment (start 61.699999 21.745) (end 61.699999 23.19) (width 0.3) (layer "F.Cu") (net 7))
 (segment (start 61.699999 23.19) (end 61.709999 23.2) (width 0.3) (layer "F.Cu") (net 7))
 (via (at 61.709999 23.2) (size 0.6) (drill 0.3) (layers "F.Cu" "B.Cu") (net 7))
 (segment (start 61.709999 24.215) (end 62.669998 25.174999) (width 0.3) (layer "B.Cu") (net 7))
 (segment (start 61.709999 23.2) (end 61.709999 24.215) (width 0.3) (layer "B.Cu") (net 7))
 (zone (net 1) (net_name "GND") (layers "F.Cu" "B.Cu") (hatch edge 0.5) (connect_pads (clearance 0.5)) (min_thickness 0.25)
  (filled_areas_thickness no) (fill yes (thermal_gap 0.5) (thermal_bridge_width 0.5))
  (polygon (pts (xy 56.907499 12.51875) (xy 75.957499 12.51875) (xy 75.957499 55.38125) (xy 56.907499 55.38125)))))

